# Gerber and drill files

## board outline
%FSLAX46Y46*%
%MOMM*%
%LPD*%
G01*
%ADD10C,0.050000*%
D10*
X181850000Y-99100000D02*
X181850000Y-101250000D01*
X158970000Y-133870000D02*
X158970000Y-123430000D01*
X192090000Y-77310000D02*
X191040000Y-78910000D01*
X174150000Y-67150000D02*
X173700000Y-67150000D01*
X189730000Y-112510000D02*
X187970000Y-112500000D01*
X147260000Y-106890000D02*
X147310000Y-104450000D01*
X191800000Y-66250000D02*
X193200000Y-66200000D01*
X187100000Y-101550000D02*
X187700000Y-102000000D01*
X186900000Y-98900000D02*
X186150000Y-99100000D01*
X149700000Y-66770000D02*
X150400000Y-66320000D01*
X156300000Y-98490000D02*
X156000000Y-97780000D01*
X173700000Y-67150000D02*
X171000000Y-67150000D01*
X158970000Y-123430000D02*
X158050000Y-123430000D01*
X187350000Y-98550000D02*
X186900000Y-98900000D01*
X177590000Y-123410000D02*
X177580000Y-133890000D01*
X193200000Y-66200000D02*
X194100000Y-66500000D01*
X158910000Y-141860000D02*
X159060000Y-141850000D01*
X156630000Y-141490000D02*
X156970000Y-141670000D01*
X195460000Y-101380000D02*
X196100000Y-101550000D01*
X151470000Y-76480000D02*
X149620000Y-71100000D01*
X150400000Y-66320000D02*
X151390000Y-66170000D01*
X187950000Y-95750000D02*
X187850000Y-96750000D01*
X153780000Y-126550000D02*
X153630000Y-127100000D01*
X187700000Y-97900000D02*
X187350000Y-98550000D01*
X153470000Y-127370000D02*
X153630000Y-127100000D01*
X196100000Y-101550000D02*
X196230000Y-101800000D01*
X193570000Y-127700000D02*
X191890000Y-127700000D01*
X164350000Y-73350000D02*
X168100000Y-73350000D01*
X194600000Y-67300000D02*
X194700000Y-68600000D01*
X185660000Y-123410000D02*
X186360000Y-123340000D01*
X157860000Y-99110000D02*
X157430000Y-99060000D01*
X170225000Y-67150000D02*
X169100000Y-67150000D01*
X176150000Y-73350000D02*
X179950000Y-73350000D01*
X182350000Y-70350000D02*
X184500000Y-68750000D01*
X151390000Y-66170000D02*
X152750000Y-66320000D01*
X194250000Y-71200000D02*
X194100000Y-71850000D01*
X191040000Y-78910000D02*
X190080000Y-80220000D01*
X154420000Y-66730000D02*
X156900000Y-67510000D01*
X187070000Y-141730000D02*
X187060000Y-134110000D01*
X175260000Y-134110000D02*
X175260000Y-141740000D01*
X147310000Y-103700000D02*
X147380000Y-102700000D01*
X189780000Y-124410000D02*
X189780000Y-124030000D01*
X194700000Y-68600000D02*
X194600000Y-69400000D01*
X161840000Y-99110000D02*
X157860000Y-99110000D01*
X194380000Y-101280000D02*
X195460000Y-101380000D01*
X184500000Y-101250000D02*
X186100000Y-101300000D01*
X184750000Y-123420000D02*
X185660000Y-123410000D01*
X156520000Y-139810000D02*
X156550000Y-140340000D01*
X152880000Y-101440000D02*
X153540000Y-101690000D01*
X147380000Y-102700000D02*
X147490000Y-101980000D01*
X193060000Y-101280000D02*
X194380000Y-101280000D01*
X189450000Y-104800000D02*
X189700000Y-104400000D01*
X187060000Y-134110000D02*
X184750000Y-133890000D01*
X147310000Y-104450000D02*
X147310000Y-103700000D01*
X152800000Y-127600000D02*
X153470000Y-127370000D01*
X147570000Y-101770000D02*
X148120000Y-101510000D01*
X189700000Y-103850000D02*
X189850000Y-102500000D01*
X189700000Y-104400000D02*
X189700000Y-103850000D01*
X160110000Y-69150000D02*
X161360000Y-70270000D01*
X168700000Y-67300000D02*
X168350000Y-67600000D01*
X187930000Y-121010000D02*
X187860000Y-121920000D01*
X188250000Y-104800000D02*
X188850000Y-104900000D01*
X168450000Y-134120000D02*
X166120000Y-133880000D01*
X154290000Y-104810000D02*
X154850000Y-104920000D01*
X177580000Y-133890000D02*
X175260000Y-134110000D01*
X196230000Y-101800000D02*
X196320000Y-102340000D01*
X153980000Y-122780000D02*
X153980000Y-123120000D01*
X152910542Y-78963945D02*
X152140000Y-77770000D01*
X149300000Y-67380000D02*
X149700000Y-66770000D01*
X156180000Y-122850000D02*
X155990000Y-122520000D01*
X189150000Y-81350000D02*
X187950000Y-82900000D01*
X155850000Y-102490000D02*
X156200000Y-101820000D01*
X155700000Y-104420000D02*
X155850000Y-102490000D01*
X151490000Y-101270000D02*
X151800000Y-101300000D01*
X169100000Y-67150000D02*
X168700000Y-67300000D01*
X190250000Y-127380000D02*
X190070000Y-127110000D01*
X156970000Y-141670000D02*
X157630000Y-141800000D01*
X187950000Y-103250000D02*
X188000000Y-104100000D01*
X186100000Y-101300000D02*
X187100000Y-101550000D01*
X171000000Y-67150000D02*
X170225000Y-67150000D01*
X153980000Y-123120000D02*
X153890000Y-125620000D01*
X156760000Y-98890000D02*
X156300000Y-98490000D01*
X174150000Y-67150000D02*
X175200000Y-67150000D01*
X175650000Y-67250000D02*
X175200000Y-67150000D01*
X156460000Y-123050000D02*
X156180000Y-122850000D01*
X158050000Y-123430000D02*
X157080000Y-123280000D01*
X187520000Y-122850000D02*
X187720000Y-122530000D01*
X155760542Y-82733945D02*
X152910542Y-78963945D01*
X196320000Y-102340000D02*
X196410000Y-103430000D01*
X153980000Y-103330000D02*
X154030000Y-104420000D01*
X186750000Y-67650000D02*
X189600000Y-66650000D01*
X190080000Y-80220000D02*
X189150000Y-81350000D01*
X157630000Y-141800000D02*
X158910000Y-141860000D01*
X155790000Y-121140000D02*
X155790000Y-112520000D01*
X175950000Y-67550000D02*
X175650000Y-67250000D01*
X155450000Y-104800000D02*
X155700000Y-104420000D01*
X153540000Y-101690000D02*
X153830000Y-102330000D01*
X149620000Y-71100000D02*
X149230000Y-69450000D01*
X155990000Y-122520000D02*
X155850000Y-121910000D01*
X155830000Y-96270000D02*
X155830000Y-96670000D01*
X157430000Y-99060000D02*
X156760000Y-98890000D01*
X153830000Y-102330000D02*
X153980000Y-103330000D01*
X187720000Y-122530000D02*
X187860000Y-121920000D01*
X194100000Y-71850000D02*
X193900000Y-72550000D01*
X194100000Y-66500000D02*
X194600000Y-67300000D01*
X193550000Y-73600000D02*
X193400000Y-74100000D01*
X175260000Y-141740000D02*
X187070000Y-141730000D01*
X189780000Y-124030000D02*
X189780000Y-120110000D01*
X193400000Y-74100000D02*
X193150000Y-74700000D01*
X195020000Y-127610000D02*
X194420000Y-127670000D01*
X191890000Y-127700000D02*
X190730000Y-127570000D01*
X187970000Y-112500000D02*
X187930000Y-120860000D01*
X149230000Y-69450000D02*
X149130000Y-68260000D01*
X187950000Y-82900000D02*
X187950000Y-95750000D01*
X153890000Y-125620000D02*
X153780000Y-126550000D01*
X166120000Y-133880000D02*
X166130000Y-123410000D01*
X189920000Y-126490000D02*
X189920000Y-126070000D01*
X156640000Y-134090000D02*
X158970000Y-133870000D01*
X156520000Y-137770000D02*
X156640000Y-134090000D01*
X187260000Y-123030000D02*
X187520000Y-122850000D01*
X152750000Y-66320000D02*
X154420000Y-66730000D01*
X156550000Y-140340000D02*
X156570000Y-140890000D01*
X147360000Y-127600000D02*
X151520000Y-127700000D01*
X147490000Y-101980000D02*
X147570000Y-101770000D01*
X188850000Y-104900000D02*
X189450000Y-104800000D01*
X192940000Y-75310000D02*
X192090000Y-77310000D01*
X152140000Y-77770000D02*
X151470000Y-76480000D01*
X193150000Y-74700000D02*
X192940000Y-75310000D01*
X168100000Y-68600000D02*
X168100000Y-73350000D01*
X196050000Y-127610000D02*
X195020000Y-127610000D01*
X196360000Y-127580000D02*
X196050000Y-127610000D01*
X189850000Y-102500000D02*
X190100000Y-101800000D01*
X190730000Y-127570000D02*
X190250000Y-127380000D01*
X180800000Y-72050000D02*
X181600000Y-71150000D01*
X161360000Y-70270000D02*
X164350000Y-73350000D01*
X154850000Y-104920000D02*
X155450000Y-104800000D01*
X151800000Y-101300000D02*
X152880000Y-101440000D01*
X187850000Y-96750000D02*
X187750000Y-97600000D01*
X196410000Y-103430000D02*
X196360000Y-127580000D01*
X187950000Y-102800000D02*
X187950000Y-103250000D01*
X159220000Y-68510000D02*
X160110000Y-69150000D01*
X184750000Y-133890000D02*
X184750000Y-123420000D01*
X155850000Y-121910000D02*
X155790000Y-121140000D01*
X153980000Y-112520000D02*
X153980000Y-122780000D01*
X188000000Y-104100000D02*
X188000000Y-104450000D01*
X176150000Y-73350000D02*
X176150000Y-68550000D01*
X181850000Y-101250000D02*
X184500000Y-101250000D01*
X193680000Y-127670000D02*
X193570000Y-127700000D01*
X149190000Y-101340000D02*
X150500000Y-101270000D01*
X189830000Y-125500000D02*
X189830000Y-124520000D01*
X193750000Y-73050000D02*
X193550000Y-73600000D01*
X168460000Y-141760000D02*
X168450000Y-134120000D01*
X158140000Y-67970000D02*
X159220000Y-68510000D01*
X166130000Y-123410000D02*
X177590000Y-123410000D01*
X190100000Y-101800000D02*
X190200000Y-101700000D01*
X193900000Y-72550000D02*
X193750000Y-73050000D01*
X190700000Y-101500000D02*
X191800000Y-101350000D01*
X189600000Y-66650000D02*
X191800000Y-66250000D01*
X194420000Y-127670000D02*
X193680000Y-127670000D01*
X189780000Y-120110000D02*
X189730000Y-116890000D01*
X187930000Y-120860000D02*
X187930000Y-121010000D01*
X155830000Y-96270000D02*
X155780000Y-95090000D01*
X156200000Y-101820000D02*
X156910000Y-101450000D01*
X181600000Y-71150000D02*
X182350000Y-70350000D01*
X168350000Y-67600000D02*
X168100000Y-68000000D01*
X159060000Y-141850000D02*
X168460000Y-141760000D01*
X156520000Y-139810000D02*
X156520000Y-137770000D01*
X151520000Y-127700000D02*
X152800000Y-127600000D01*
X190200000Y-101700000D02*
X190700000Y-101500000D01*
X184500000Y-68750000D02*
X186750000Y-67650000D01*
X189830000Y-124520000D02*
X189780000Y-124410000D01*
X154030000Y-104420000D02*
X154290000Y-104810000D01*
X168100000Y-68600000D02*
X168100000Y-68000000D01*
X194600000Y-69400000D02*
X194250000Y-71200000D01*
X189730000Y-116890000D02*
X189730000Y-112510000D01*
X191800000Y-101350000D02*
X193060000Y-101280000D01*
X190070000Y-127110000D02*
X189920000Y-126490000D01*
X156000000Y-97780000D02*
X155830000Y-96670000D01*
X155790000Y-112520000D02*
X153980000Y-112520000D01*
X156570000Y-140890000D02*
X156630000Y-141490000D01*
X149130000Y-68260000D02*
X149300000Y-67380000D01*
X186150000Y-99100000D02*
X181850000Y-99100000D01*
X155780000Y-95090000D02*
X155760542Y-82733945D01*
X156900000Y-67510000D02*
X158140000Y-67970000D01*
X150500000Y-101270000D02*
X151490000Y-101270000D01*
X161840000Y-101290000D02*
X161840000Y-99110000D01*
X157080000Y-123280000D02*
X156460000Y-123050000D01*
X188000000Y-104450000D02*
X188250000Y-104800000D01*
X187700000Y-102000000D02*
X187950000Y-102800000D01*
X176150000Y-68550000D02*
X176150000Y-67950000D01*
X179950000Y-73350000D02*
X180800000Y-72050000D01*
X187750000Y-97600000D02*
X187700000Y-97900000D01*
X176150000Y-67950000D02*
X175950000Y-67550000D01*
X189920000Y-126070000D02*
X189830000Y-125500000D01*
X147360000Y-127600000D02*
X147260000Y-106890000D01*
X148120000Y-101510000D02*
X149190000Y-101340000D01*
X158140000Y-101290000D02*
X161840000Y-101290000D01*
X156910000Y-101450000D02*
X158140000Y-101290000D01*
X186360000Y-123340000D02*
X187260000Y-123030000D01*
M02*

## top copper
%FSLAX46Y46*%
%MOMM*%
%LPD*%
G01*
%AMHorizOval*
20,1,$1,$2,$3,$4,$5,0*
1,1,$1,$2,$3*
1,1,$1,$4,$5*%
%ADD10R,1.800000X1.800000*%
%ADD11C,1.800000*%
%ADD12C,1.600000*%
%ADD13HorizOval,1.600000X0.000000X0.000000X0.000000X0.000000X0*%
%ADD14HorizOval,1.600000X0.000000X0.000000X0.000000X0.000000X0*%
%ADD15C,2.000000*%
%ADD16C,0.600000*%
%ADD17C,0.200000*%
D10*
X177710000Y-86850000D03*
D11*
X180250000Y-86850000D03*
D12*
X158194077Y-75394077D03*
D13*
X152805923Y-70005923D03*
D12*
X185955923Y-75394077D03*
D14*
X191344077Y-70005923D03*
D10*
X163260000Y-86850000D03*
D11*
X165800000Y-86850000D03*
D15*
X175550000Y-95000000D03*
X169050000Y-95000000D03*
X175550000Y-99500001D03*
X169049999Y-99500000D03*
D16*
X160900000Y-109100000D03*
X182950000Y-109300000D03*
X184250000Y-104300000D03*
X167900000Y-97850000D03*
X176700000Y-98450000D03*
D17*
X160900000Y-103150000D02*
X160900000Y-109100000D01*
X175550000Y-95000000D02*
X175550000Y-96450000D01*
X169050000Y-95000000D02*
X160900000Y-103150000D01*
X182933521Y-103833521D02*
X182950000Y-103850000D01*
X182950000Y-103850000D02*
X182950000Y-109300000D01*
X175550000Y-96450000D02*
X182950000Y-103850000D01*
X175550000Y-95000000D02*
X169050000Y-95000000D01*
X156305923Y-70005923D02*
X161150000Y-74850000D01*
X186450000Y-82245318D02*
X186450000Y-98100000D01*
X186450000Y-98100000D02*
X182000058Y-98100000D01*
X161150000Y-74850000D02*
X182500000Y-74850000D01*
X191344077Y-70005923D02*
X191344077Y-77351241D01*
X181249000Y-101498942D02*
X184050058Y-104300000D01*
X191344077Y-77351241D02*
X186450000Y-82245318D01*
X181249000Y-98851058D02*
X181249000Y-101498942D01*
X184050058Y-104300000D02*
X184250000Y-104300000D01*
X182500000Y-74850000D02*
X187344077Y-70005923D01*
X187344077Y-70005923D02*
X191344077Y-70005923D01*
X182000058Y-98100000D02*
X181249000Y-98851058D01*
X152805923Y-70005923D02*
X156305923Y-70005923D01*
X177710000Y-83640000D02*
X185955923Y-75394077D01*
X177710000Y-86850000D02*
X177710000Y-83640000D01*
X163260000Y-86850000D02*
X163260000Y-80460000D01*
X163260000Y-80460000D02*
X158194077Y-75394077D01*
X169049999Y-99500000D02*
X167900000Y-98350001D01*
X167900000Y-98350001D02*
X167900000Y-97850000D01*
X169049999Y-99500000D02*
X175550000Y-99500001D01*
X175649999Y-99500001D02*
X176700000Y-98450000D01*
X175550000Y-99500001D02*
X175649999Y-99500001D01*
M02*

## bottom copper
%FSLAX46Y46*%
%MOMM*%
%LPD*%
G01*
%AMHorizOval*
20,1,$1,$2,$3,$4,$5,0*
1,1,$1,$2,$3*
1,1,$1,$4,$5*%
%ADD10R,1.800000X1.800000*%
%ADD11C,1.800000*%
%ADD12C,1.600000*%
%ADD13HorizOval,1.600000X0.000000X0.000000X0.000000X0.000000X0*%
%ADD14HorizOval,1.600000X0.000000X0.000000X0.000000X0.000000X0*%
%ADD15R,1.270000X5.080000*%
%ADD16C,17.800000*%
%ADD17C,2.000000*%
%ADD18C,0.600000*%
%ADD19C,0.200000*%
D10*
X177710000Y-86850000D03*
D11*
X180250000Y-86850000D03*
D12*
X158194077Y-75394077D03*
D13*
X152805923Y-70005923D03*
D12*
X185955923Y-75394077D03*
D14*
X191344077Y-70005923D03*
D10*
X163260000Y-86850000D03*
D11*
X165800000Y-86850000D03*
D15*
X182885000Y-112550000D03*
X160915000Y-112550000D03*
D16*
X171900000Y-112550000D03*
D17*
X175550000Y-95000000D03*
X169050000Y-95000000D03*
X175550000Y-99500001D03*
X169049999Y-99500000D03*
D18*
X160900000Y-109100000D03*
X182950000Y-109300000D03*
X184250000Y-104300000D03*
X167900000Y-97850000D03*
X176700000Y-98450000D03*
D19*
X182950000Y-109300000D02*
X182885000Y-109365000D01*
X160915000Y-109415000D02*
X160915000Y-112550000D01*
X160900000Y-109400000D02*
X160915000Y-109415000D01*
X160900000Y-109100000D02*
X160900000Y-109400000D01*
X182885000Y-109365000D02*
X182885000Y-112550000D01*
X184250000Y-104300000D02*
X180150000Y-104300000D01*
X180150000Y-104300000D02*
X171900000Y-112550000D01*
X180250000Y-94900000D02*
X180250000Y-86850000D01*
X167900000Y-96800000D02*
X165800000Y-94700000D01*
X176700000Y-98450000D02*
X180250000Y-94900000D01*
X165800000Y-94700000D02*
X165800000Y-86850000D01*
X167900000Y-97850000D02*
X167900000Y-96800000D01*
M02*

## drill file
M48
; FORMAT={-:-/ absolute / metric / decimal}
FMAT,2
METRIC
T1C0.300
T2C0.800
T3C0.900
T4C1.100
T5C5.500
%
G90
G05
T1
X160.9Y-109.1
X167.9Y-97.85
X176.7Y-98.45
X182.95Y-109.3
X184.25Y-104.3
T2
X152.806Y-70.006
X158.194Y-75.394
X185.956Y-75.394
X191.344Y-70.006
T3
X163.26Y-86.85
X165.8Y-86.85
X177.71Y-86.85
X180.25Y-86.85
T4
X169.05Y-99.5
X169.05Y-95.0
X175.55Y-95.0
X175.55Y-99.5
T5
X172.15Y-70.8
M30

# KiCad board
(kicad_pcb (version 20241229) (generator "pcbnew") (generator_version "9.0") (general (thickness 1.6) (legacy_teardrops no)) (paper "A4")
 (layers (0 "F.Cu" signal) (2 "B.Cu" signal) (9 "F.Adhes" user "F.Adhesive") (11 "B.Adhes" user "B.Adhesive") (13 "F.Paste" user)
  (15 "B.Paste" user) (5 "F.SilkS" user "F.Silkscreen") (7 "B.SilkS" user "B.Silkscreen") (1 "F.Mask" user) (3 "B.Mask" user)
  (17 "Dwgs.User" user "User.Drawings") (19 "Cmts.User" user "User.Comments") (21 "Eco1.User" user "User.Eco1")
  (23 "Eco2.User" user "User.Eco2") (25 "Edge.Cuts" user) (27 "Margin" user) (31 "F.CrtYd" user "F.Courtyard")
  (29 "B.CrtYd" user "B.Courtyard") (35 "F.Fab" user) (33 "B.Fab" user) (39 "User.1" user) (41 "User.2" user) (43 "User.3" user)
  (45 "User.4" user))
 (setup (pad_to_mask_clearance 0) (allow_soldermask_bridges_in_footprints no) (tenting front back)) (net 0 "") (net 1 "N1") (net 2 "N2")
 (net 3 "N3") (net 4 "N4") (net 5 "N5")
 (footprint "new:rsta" (layer "F.Cu") (at 170.3 106.931432)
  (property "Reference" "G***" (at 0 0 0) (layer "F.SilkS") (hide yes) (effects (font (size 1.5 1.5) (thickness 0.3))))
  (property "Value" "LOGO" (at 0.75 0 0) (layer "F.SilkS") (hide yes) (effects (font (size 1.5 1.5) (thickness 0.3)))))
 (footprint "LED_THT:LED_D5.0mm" (layer "F.Cu") (at 177.71 86.85)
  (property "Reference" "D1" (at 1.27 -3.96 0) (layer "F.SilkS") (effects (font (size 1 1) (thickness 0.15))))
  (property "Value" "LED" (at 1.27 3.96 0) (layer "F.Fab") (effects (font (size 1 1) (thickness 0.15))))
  (pad "1" thru_hole rect (at 0 0) (size 1.8 1.8) (drill 0.9) (layers "*.Cu" "*.Mask") (remove_unused_layers no) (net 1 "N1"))
  (pad "2" thru_hole circle (at 2.54 0) (size 1.8 1.8) (drill 0.9) (layers "*.Cu" "*.Mask") (remove_unused_layers no) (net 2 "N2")))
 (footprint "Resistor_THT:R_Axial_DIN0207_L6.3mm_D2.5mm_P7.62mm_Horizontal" (layer "F.Cu") (at 158.194077 75.394077 135)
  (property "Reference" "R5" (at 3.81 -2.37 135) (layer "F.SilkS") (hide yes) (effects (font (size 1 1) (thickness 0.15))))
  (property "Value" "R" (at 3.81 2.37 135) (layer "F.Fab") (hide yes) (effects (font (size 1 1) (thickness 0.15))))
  (pad "1" thru_hole circle (at 0 0 135) (size 1.6 1.6) (drill 0.8) (layers "*.Cu" "*.Mask") (remove_unused_layers no) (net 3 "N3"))
  (pad "2" thru_hole oval (at 7.62 0 135) (size 1.6 1.6) (drill 0.8) (layers "*.Cu" "*.Mask") (remove_unused_layers no) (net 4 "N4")))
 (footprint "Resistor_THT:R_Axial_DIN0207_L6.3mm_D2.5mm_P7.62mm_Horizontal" (layer "F.Cu") (at 185.955923 75.394077 45)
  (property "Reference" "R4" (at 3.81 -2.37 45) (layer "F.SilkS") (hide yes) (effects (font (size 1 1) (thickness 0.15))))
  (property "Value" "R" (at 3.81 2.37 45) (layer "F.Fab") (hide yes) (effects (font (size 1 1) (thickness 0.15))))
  (pad "1" thru_hole circle (at 0 0 45) (size 1.6 1.6) (drill 0.8) (layers "*.Cu" "*.Mask") (remove_unused_layers no) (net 1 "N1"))
  (pad "2" thru_hole oval (at 7.62 0 45) (size 1.6 1.6) (drill 0.8) (layers "*.Cu" "*.Mask") (remove_unused_layers no) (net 4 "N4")))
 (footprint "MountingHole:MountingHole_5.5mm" (layer "F.Cu") (at 172.15 70.8)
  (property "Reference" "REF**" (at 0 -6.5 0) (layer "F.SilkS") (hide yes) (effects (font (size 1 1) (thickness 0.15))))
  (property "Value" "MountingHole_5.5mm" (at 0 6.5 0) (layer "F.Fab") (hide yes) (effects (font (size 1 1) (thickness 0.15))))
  (pad "" np_thru_hole circle (at 0 0) (size 5.5 5.5) (drill 5.5) (layers "*.Cu" "*.Mask")))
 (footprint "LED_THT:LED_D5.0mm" (layer "F.Cu") (at 163.26 86.85)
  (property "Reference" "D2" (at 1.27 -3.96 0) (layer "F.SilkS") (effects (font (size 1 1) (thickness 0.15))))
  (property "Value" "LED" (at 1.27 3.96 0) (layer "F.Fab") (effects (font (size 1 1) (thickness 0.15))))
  (pad "1" thru_hole rect (at 0 0) (size 1.8 1.8) (drill 0.9) (layers "*.Cu" "*.Mask") (remove_unused_layers no) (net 3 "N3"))
  (pad "2" thru_hole circle (at 2.54 0) (size 1.8 1.8) (drill 0.9) (layers "*.Cu" "*.Mask") (remove_unused_layers no) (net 2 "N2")))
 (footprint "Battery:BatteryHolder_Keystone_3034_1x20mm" (layer "B.Cu") (at 171.9 112.55 180)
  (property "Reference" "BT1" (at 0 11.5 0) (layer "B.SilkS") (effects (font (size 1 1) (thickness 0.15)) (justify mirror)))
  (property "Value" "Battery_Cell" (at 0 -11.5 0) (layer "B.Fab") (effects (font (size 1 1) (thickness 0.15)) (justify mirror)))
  (pad "1" smd rect (at -10.985 0 180) (size 1.27 5.08) (layers "B.Cu" "B.Mask" "B.Paste") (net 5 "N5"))
  (pad "1" smd rect (at 10.985 0 180) (size 1.27 5.08) (layers "B.Cu" "B.Mask" "B.Paste") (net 5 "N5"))
  (pad "2" smd circle (at 0 0 180) (size 17.8 17.8) (layers "B.Cu" "B.Mask") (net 4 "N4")))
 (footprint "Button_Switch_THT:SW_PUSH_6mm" (layer "B.Cu") (at 175.55 95 180)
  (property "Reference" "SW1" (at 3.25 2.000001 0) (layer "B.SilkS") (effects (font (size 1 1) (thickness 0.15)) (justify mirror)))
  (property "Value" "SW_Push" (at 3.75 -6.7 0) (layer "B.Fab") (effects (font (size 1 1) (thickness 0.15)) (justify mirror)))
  (pad "1" thru_hole circle (at 0 0 90) (size 2 2) (drill 1.1) (layers "*.Cu" "*.Mask") (remove_unused_layers no) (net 5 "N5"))
  (pad "1" thru_hole circle (at 6.5 0 90) (size 2 2) (drill 1.1) (layers "*.Cu" "*.Mask") (remove_unused_layers no) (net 5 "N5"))
  (pad "2" thru_hole circle (at 0 -4.500001 90) (size 2 2) (drill 1.1) (layers "*.Cu" "*.Mask") (remove_unused_layers no) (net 2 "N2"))
  (pad "2" thru_hole circle (at 6.500001 -4.5 90) (size 2 2) (drill 1.1) (layers "*.Cu" "*.Mask") (remove_unused_layers no) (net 2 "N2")))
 (gr_line (start 181.85 99.1) (end 181.85 101.25) (stroke (width 0.05) (type default)) (layer "Edge.Cuts"))
 (gr_line (start 158.97 133.87) (end 158.97 123.43) (stroke (width 0.05) (type default)) (layer "Edge.Cuts"))
 (gr_line (start 192.09 77.31) (end 191.04 78.91) (stroke (width 0.05) (type default)) (layer "Edge.Cuts"))
 (gr_line (start 174.15 67.15) (end 173.7 67.15) (stroke (width 0.05) (type default)) (layer "Edge.Cuts"))
 (gr_line (start 189.73 112.51) (end 187.97 112.5) (stroke (width 0.05) (type default)) (layer "Edge.Cuts"))
 (gr_line (start 147.26 106.89) (end 147.31 104.45) (stroke (width 0.05) (type default)) (layer "Edge.Cuts"))
 (gr_line (start 191.8 66.25) (end 193.2 66.2) (stroke (width 0.05) (type default)) (layer "Edge.Cuts"))
 (gr_line (start 187.1 101.55) (end 187.7 102) (stroke (width 0.05) (type default)) (layer "Edge.Cuts"))
 (gr_line (start 186.9 98.9) (end 186.15 99.1) (stroke (width 0.05) (type default)) (layer "Edge.Cuts"))
 (gr_line (start 149.7 66.77) (end 150.4 66.32) (stroke (width 0.05) (type default)) (layer "Edge.Cuts"))
 (gr_line (start 156.3 98.49) (end 156 97.78) (stroke (width 0.05) (type default)) (layer "Edge.Cuts"))
 (gr_line (start 173.7 67.15) (end 171 67.15) (stroke (width 0.05) (type default)) (layer "Edge.Cuts"))
 (gr_line (start 158.97 123.43) (end 158.05 123.43) (stroke (width 0.05) (type default)) (layer "Edge.Cuts"))
 (gr_line (start 187.35 98.55) (end 186.9 98.9) (stroke (width 0.05) (type default)) (layer "Edge.Cuts"))
 (gr_line (start 177.59 123.41) (end 177.58 133.89) (stroke (width 0.05) (type default)) (layer "Edge.Cuts"))
 (gr_line (start 193.2 66.2) (end 194.1 66.5) (stroke (width 0.05) (type default)) (layer "Edge.Cuts"))
 (gr_line (start 158.91 141.86) (end 159.06 141.85) (stroke (width 0.05) (type default)) (layer "Edge.Cuts"))
 (gr_line (start 156.63 141.49) (end 156.97 141.67) (stroke (width 0.05) (type default)) (layer "Edge.Cuts"))
 (gr_line (start 195.46 101.38) (end 196.1 101.55) (stroke (width 0.05) (type default)) (layer "Edge.Cuts"))
 (gr_line (start 151.47 76.48) (end 149.62 71.1) (stroke (width 0.05) (type default)) (layer "Edge.Cuts"))
 (gr_line (start 150.4 66.32) (end 151.39 66.17) (stroke (width 0.05) (type default)) (layer "Edge.Cuts"))
 (gr_line (start 187.95 95.75) (end 187.85 96.75) (stroke (width 0.05) (type default)) (layer "Edge.Cuts"))
 (gr_line (start 153.78 126.55) (end 153.63 127.1) (stroke (width 0.05) (type default)) (layer "Edge.Cuts"))
 (gr_line (start 187.7 97.9) (end 187.35 98.55) (stroke (width 0.05) (type default)) (layer "Edge.Cuts"))
 (gr_line (start 153.47 127.37) (end 153.63 127.1) (stroke (width 0.05) (type default)) (layer "Edge.Cuts"))
 (gr_line (start 196.1 101.55) (end 196.23 101.8) (stroke (width 0.05) (type default)) (layer "Edge.Cuts"))
 (gr_line (start 193.57 127.7) (end 191.89 127.7) (stroke (width 0.05) (type default)) (layer "Edge.Cuts"))
 (gr_line (start 164.35 73.35) (end 168.1 73.35) (stroke (width 0.05) (type default)) (layer "Edge.Cuts"))
 (gr_line (start 194.6 67.3) (end 194.7 68.6) (stroke (width 0.05) (type default)) (layer "Edge.Cuts"))
 (gr_line (start 185.66 123.41) (end 186.36 123.34) (stroke (width 0.05) (type default)) (layer "Edge.Cuts"))
 (gr_line (start 157.86 99.11) (end 157.43 99.06) (stroke (width 0.05) (type default)) (layer "Edge.Cuts"))
 (gr_line (start 170.225 67.15) (end 169.1 67.15) (stroke (width 0.05) (type default)) (layer "Edge.Cuts"))
 (gr_line (start 176.15 73.35) (end 179.95 73.35) (stroke (width 0.05) (type default)) (layer "Edge.Cuts"))
 (gr_line (start 182.35 70.35) (end 184.5 68.75) (stroke (width 0.05) (type default)) (layer "Edge.Cuts"))
 (gr_line (start 151.39 66.17) (end 152.75 66.32) (stroke (width 0.05) (type default)) (layer "Edge.Cuts"))
 (gr_line (start 194.25 71.2) (end 194.1 71.85) (stroke (width 0.05) (type default)) (layer "Edge.Cuts"))
 (gr_line (start 191.04 78.91) (end 190.08 80.22) (stroke (width 0.05) (type default)) (layer "Edge.Cuts"))
 (gr_line (start 154.42 66.73) (end 156.9 67.51) (stroke (width 0.05) (type default)) (layer "Edge.Cuts"))
 (gr_line (start 187.07 141.73) (end 187.06 134.11) (stroke (width 0.05) (type default)) (layer "Edge.Cuts"))
 (gr_line (start 175.26 134.11) (end 175.26 141.74) (stroke (width 0.05) (type default)) (layer "Edge.Cuts"))
 (gr_line (start 147.31 103.7) (end 147.38 102.7) (stroke (width 0.05) (type default)) (layer "Edge.Cuts"))
 (gr_line (start 189.78 124.41) (end 189.78 124.03) (stroke (width 0.05) (type default)) (layer "Edge.Cuts"))
 (gr_line (start 194.7 68.6) (end 194.6 69.4) (stroke (width 0.05) (type default)) (layer "Edge.Cuts"))
 (gr_line (start 161.84 99.11) (end 157.86 99.11) (stroke (width 0.05) (type default)) (layer "Edge.Cuts"))
 (gr_line (start 194.38 101.28) (end 195.46 101.38) (stroke (width 0.05) (type default)) (layer "Edge.Cuts"))
 (gr_line (start 184.5 101.25) (end 186.1 101.3) (stroke (width 0.05) (type default)) (layer "Edge.Cuts"))
 (gr_line (start 184.75 123.42) (end 185.66 123.41) (stroke (width 0.05) (type default)) (layer "Edge.Cuts"))
 (gr_line (start 156.52 139.81) (end 156.55 140.34) (stroke (width 0.05) (type default)) (layer "Edge.Cuts"))
 (gr_line (start 152.88 101.44) (end 153.54 101.69) (stroke (width 0.05) (type default)) (layer "Edge.Cuts"))
 (gr_line (start 147.38 102.7) (end 147.49 101.98) (stroke (width 0.05) (type default)) (layer "Edge.Cuts"))
 (gr_line (start 193.06 101.28) (end 194.38 101.28) (stroke (width 0.05) (type default)) (layer "Edge.Cuts"))
 (gr_line (start 189.45 104.8) (end 189.7 104.4) (stroke (width 0.05) (type default)) (layer "Edge.Cuts"))
 (gr_line (start 187.06 134.11) (end 184.75 133.89) (stroke (width 0.05) (type default)) (layer "Edge.Cuts"))
 (gr_line (start 147.31 104.45) (end 147.31 103.7) (stroke (width 0.05) (type default)) (layer "Edge.Cuts"))
 (gr_line (start 152.8 127.6) (end 153.47 127.37) (stroke (width 0.05) (type default)) (layer "Edge.Cuts"))
 (gr_line (start 147.57 101.77) (end 148.12 101.51) (stroke (width 0.05) (type default)) (layer "Edge.Cuts"))
 (gr_line (start 189.7 103.85) (end 189.85 102.5) (stroke (width 0.05) (type default)) (layer "Edge.Cuts"))
 (gr_line (start 189.7 104.4) (end 189.7 103.85) (stroke (width 0.05) (type default)) (layer "Edge.Cuts"))
 (gr_line (start 160.11 69.15) (end 161.36 70.27) (stroke (width 0.05) (type default)) (layer "Edge.Cuts"))
 (gr_line (start 168.7 67.3) (end 168.35 67.6) (stroke (width 0.05) (type default)) (layer "Edge.Cuts"))
 (gr_line (start 187.93 121.01) (end 187.86 121.92) (stroke (width 0.05) (type default)) (layer "Edge.Cuts"))
 (gr_line (start 188.25 104.8) (end 188.85 104.9) (stroke (width 0.05) (type default)) (layer "Edge.Cuts"))
 (gr_line (start 168.45 134.12) (end 166.12 133.88) (stroke (width 0.05) (type default)) (layer "Edge.Cuts"))
 (gr_line (start 154.29 104.81) (end 154.85 104.92) (stroke (width 0.05) (type default)) (layer "Edge.Cuts"))
 (gr_line (start 177.58 133.89) (end 175.26 134.11) (stroke (width 0.05) (type default)) (layer "Edge.Cuts"))
 (gr_line (start 196.23 101.8) (end 196.32 102.34) (stroke (width 0.05) (type default)) (layer "Edge.Cuts"))
 (gr_line (start 153.98 122.78) (end 153.98 123.12) (stroke (width 0.05) (type default)) (layer "Edge.Cuts"))
 (gr_line (start 152.910542 78.963945) (end 152.14 77.77) (stroke (width 0.05) (type default)) (layer "Edge.Cuts"))
 (gr_line (start 149.3 67.38) (end 149.7 66.77) (stroke (width 0.05) (type default)) (layer "Edge.Cuts"))
 (gr_line (start 156.18 122.85) (end 155.99 122.52) (stroke (width 0.05) (type default)) (layer "Edge.Cuts"))
 (gr_line (start 189.15 81.35) (end 187.95 82.9) (stroke (width 0.05) (type default)) (layer "Edge.Cuts"))
 (gr_line (start 155.85 102.49) (end 156.2 101.82) (stroke (width 0.05) (type default)) (layer "Edge.Cuts"))
 (gr_line (start 155.7 104.42) (end 155.85 102.49) (stroke (width 0.05) (type default)) (layer "Edge.Cuts"))
 (gr_line (start 151.49 101.27) (end 151.8 101.3) (stroke (width 0.05) (type default)) (layer "Edge.Cuts"))
 (gr_line (start 169.1 67.15) (end 168.7 67.3) (stroke (width 0.05) (type default)) (layer "Edge.Cuts"))
 (gr_line (start 190.25 127.38) (end 190.07 127.11) (stroke (width 0.05) (type default)) (layer "Edge.Cuts"))
 (gr_line (start 156.97 141.67) (end 157.63 141.8) (stroke (width 0.05) (type default)) (layer "Edge.Cuts"))
 (gr_line (start 187.95 103.25) (end 188 104.1) (stroke (width 0.05) (type default)) (layer "Edge.Cuts"))
 (gr_line (start 186.1 101.3) (end 187.1 101.55) (stroke (width 0.05) (type default)) (layer "Edge.Cuts"))
 (gr_line (start 171 67.15) (end 170.225 67.15) (stroke (width 0.05) (type default)) (layer "Edge.Cuts"))
 (gr_line (start 153.98 123.12) (end 153.89 125.62) (stroke (width 0.05) (type default)) (layer "Edge.Cuts"))
 (gr_line (start 156.76 98.89) (end 156.3 98.49) (stroke (width 0.05) (type default)) (layer "Edge.Cuts"))
 (gr_line (start 174.15 67.15) (end 175.2 67.15) (stroke (width 0.05) (type default)) (layer "Edge.Cuts"))
 (gr_line (start 175.65 67.25) (end 175.2 67.15) (stroke (width 0.05) (type default)) (layer "Edge.Cuts"))
 (gr_line (start 156.46 123.05) (end 156.18 122.85) (stroke (width 0.05) (type default)) (layer "Edge.Cuts"))
 (gr_line (start 158.05 123.43) (end 157.08 123.28) (stroke (width 0.05) (type default)) (layer "Edge.Cuts"))
 (gr_line (start 187.52 122.85) (end 187.72 122.53) (stroke (width 0.05) (type default)) (layer "Edge.Cuts"))
 (gr_line (start 155.760542 82.733945) (end 152.910542 78.963945) (stroke (width 0.05) (type default)) (layer "Edge.Cuts"))
 (gr_line (start 196.32 102.34) (end 196.41 103.43) (stroke (width 0.05) (type default)) (layer "Edge.Cuts"))
 (gr_line (start 153.98 103.33) (end 154.03 104.42) (stroke (width 0.05) (type default)) (layer "Edge.Cuts"))
 (gr_line (start 186.75 67.65) (end 189.6 66.65) (stroke (width 0.05) (type default)) (layer "Edge.Cuts"))
 (gr_line (start 190.08 80.22) (end 189.15 81.35) (stroke (width 0.05) (type default)) (layer "Edge.Cuts"))
 (gr_line (start 157.63 141.8) (end 158.91 141.86) (stroke (width 0.05) (type default)) (layer "Edge.Cuts"))
 (gr_line (start 155.79 121.14) (end 155.79 112.52) (stroke (width 0.05) (type default)) (layer "Edge.Cuts"))
 (gr_line (start 175.95 67.55) (end 175.65 67.25) (stroke (width 0.05) (type default)) (layer "Edge.Cuts"))
 (gr_line (start 155.45 104.8) (end 155.7 104.42) (stroke (width 0.05) (type default)) (layer "Edge.Cuts"))
 (gr_line (start 153.54 101.69) (end 153.83 102.33) (stroke (width 0.05) (type default)) (layer "Edge.Cuts"))
 (gr_line (start 149.62 71.1) (end 149.23 69.45) (stroke (width 0.05) (type default)) (layer "Edge.Cuts"))
 (gr_line (start 155.99 122.52) (end 155.85 121.91) (stroke (width 0.05) (type default)) (layer "Edge.Cuts"))
 (gr_line (start 155.83 96.27) (end 155.83 96.67) (stroke (width 0.05) (type default)) (layer "Edge.Cuts"))
 (gr_line (start 157.43 99.06) (end 156.76 98.89) (stroke (width 0.05) (type default)) (layer "Edge.Cuts"))
 (gr_line (start 153.83 102.33) (end 153.98 103.33) (stroke (width 0.05) (type default)) (layer "Edge.Cuts"))
 (gr_line (start 187.72 122.53) (end 187.86 121.92) (stroke (width 0.05) (type default)) (layer "Edge.Cuts"))
 (gr_line (start 194.1 71.85) (end 193.9 72.55) (stroke (width 0.05) (type default)) (layer "Edge.Cuts"))
 (gr_line (start 194.1 66.5) (end 194.6 67.3) (stroke (width 0.05) (type default)) (layer "Edge.Cuts"))
 (gr_line (start 193.55 73.6) (end 193.4 74.1) (stroke (width 0.05) (type default)) (layer "Edge.Cuts"))
 (gr_line (start 175.26 141.74) (end 187.07 141.73) (stroke (width 0.05) (type default)) (layer "Edge.Cuts"))
 (gr_line (start 189.78 124.03) (end 189.78 120.11) (stroke (width 0.05) (type default)) (layer "Edge.Cuts"))
 (gr_line (start 193.4 74.1) (end 193.15 74.7) (stroke (width 0.05) (type default)) (layer "Edge.Cuts"))
 (gr_line (start 195.02 127.61) (end 194.42 127.67) (stroke (width 0.05) (type default)) (layer "Edge.Cuts"))
 (gr_line (start 191.89 127.7) (end 190.73 127.57) (stroke (width 0.05) (type default)) (layer "Edge.Cuts"))
 (gr_line (start 187.97 112.5) (end 187.93 120.86) (stroke (width 0.05) (type default)) (layer "Edge.Cuts"))
 (gr_line (start 149.23 69.45) (end 149.13 68.26) (stroke (width 0.05) (type default)) (layer "Edge.Cuts"))
 (gr_line (start 187.95 82.9) (end 187.95 95.75) (stroke (width 0.05) (type default)) (layer "Edge.Cuts"))
 (gr_line (start 153.89 125.62) (end 153.78 126.55) (stroke (width 0.05) (type default)) (layer "Edge.Cuts"))
 (gr_line (start 166.12 133.88) (end 166.13 123.41) (stroke (width 0.05) (type default)) (layer "Edge.Cuts"))
 (gr_line (start 189.92 126.49) (end 189.92 126.07) (stroke (width 0.05) (type default)) (layer "Edge.Cuts"))
 (gr_line (start 156.64 134.09) (end 158.97 133.87) (stroke (width 0.05) (type default)) (layer "Edge.Cuts"))
 (gr_line (start 156.52 137.77) (end 156.64 134.09) (stroke (width 0.05) (type default)) (layer "Edge.Cuts"))
 (gr_line (start 187.26 123.03) (end 187.52 122.85) (stroke (width 0.05) (type default)) (layer "Edge.Cuts"))
 (gr_line (start 152.75 66.32) (end 154.42 66.73) (stroke (width 0.05) (type default)) (layer "Edge.Cuts"))
 (gr_line (start 156.55 140.34) (end 156.57 140.89) (stroke (width 0.05) (type default)) (layer "Edge.Cuts"))
 (gr_line (start 147.36 127.6) (end 151.52 127.7) (stroke (width 0.05) (type default)) (layer "Edge.Cuts"))
 (gr_line (start 147.49 101.98) (end 147.57 101.77) (stroke (width 0.05) (type default)) (layer "Edge.Cuts"))
 (gr_line (start 188.85 104.9) (end 189.45 104.8) (stroke (width 0.05) (type default)) (layer "Edge.Cuts"))
 (gr_line (start 192.94 75.31) (end 192.09 77.31) (stroke (width 0.05) (type default)) (layer "Edge.Cuts"))
 (gr_line (start 152.14 77.77) (end 151.47 76.48) (stroke (width 0.05) (type default)) (layer "Edge.Cuts"))
 (gr_line (start 193.15 74.7) (end 192.94 75.31) (stroke (width 0.05) (type default)) (layer "Edge.Cuts"))
 (gr_line (start 168.1 68.6) (end 168.1 73.35) (stroke (width 0.05) (type default)) (layer "Edge.Cuts"))
 (gr_line (start 196.05 127.61) (end 195.02 127.61) (stroke (width 0.05) (type default)) (layer "Edge.Cuts"))
 (gr_line (start 196.36 127.58) (end 196.05 127.61) (stroke (width 0.05) (type default)) (layer "Edge.Cuts"))
 (gr_line (start 189.85 102.5) (end 190.1 101.8) (stroke (width 0.05) (type default)) (layer "Edge.Cuts"))
 (gr_line (start 190.73 127.57) (end 190.25 127.38) (stroke (width 0.05) (type default)) (layer "Edge.Cuts"))
 (gr_line (start 180.8 72.05) (end 181.6 71.15) (stroke (width 0.05) (type default)) (layer "Edge.Cuts"))
 (gr_line (start 161.36 70.27) (end 164.35 73.35) (stroke (width 0.05) (type default)) (layer "Edge.Cuts"))
 (gr_line (start 154.85 104.92) (end 155.45 104.8) (stroke (width 0.05) (type default)) (layer "Edge.Cuts"))
 (gr_line (start 151.8 101.3) (end 152.88 101.44) (stroke (width 0.05) (type default)) (layer "Edge.Cuts"))
 (gr_line (start 187.85 96.75) (end 187.75 97.6) (stroke (width 0.05) (type default)) (layer "Edge.Cuts"))
 (gr_line (start 196.41 103.43) (end 196.36 127.58) (stroke (width 0.05) (type default)) (layer "Edge.Cuts"))
 (gr_line (start 187.95 102.8) (end 187.95 103.25) (stroke (width 0.05) (type default)) (layer "Edge.Cuts"))
 (gr_line (start 159.22 68.51) (end 160.11 69.15) (stroke (width 0.05) (type default)) (layer "Edge.Cuts"))
 (gr_line (start 184.75 133.89) (end 184.75 123.42) (stroke (width 0.05) (type default)) (layer "Edge.Cuts"))
 (gr_line (start 155.85 121.91) (end 155.79 121.14) (stroke (width 0.05) (type default)) (layer "Edge.Cuts"))
 (gr_line (start 153.98 112.52) (end 153.98 122.78) (stroke (width 0.05) (type default)) (layer "Edge.Cuts"))
 (gr_line (start 188 104.1) (end 188 104.45) (stroke (width 0.05) (type default)) (layer "Edge.Cuts"))
 (gr_line (start 176.15 73.35) (end 176.15 68.55) (stroke (width 0.05) (type default)) (layer "Edge.Cuts"))
 (gr_line (start 181.85 101.25) (end 184.5 101.25) (stroke (width 0.05) (type default)) (layer "Edge.Cuts"))
 (gr_line (start 193.68 127.67) (end 193.57 127.7) (stroke (width 0.05) (type default)) (layer "Edge.Cuts"))
 (gr_line (start 149.19 101.34) (end 150.5 101.27) (stroke (width 0.05) (type default)) (layer "Edge.Cuts"))
 (gr_line (start 189.83 125.5) (end 189.83 124.52) (stroke (width 0.05) (type default)) (layer "Edge.Cuts"))
 (gr_line (start 193.75 73.05) (end 193.55 73.6) (stroke (width 0.05) (type default)) (layer "Edge.Cuts"))
 (gr_line (start 168.46 141.76) (end 168.45 134.12) (stroke (width 0.05) (type default)) (layer "Edge.Cuts"))
 (gr_line (start 158.14 67.97) (end 159.22 68.51) (stroke (width 0.05) (type default)) (layer "Edge.Cuts"))
 (gr_line (start 166.13 123.41) (end 177.59 123.41) (stroke (width 0.05) (type default)) (layer "Edge.Cuts"))
 (gr_line (start 190.1 101.8) (end 190.2 101.7) (stroke (width 0.05) (type default)) (layer "Edge.Cuts"))
 (gr_line (start 193.9 72.55) (end 193.75 73.05) (stroke (width 0.05) (type default)) (layer "Edge.Cuts"))
 (gr_line (start 190.7 101.5) (end 191.8 101.35) (stroke (width 0.05) (type default)) (layer "Edge.Cuts"))
 (gr_line (start 189.6 66.65) (end 191.8 66.25) (stroke (width 0.05) (type default)) (layer "Edge.Cuts"))
 (gr_line (start 194.42 127.67) (end 193.68 127.67) (stroke (width 0.05) (type default)) (layer "Edge.Cuts"))
 (gr_line (start 189.78 120.11) (end 189.73 116.89) (stroke (width 0.05) (type default)) (layer "Edge.Cuts"))
 (gr_line (start 187.93 120.86) (end 187.93 121.01) (stroke (width 0.05) (type default)) (layer "Edge.Cuts"))
 (gr_line (start 155.83 96.27) (end 155.78 95.09) (stroke (width 0.05) (type default)) (layer "Edge.Cuts"))
 (gr_line (start 156.2 101.82) (end 156.91 101.45) (stroke (width 0.05) (type default)) (layer "Edge.Cuts"))
 (gr_line (start 181.6 71.15) (end 182.35 70.35) (stroke (width 0.05) (type default)) (layer "Edge.Cuts"))
 (gr_line (start 168.35 67.6) (end 168.1 68) (stroke (width 0.05) (type default)) (layer "Edge.Cuts"))
 (gr_line (start 159.06 141.85) (end 168.46 141.76) (stroke (width 0.05) (type default)) (layer "Edge.Cuts"))
 (gr_line (start 156.52 139.81) (end 156.52 137.77) (stroke (width 0.05) (type default)) (layer "Edge.Cuts"))
 (gr_line (start 151.52 127.7) (end 152.8 127.6) (stroke (width 0.05) (type default)) (layer "Edge.Cuts"))
 (gr_line (start 190.2 101.7) (end 190.7 101.5) (stroke (width 0.05) (type default)) (layer "Edge.Cuts"))
 (gr_line (start 184.5 68.75) (end 186.75 67.65) (stroke (width 0.05) (type default)) (layer "Edge.Cuts"))
 (gr_line (start 189.83 124.52) (end 189.78 124.41) (stroke (width 0.05) (type default)) (layer "Edge.Cuts"))
 (gr_line (start 154.03 104.42) (end 154.29 104.81) (stroke (width 0.05) (type default)) (layer "Edge.Cuts"))
 (gr_line (start 168.1 68.6) (end 168.1 68) (stroke (width 0.05) (type default)) (layer "Edge.Cuts"))
 (gr_line (start 194.6 69.4) (end 194.25 71.2) (stroke (width 0.05) (type default)) (layer "Edge.Cuts"))
 (gr_line (start 189.73 116.89) (end 189.73 112.51) (stroke (width 0.05) (type default)) (layer "Edge.Cuts"))
 (gr_line (start 191.8 101.35) (end 193.06 101.28) (stroke (width 0.05) (type default)) (layer "Edge.Cuts"))
 (gr_line (start 190.07 127.11) (end 189.92 126.49) (stroke (width 0.05) (type default)) (layer "Edge.Cuts"))
 (gr_line (start 156 97.78) (end 155.83 96.67) (stroke (width 0.05) (type default)) (layer "Edge.Cuts"))
 (gr_line (start 155.79 112.52) (end 153.98 112.52) (stroke (width 0.05) (type default)) (layer "Edge.Cuts"))
 (gr_line (start 156.57 140.89) (end 156.63 141.49) (stroke (width 0.05) (type default)) (layer "Edge.Cuts"))
 (gr_line (start 149.13 68.26) (end 149.3 67.38) (stroke (width 0.05) (type default)) (layer "Edge.Cuts"))
 (gr_line (start 186.15 99.1) (end 181.85 99.1) (stroke (width 0.05) (type default)) (layer "Edge.Cuts"))
 (gr_line (start 155.78 95.09) (end 155.760542 82.733945) (stroke (width 0.05) (type default)) (layer "Edge.Cuts"))
 (gr_line (start 156.9 67.51) (end 158.14 67.97) (stroke (width 0.05) (type default)) (layer "Edge.Cuts"))
 (gr_line (start 150.5 101.27) (end 151.49 101.27) (stroke (width 0.05) (type default)) (layer "Edge.Cuts"))
 (gr_line (start 161.84 101.29) (end 161.84 99.11) (stroke (width 0.05) (type default)) (layer "Edge.Cuts"))
 (gr_line (start 157.08 123.28) (end 156.46 123.05) (stroke (width 0.05) (type default)) (layer "Edge.Cuts"))
 (gr_line (start 188 104.45) (end 188.25 104.8) (stroke (width 0.05) (type default)) (layer "Edge.Cuts"))
 (gr_line (start 187.7 102) (end 187.95 102.8) (stroke (width 0.05) (type default)) (layer "Edge.Cuts"))
 (gr_line (start 176.15 68.55) (end 176.15 67.95) (stroke (width 0.05) (type default)) (layer "Edge.Cuts"))
 (gr_line (start 179.95 73.35) (end 180.8 72.05) (stroke (width 0.05) (type default)) (layer "Edge.Cuts"))
 (gr_line (start 187.75 97.6) (end 187.7 97.9) (stroke (width 0.05) (type default)) (layer "Edge.Cuts"))
 (gr_line (start 176.15 67.95) (end 175.95 67.55) (stroke (width 0.05) (type default)) (layer "Edge.Cuts"))
 (gr_line (start 189.92 126.07) (end 189.83 125.5) (stroke (width 0.05) (type default)) (layer "Edge.Cuts"))
 (gr_line (start 147.36 127.6) (end 147.26 106.89) (stroke (width 0.05) (type default)) (layer "Edge.Cuts"))
 (gr_line (start 148.12 101.51) (end 149.19 101.34) (stroke (width 0.05) (type default)) (layer "Edge.Cuts"))
 (gr_line (start 158.14 101.29) (end 161.84 101.29) (stroke (width 0.05) (type default)) (layer "Edge.Cuts"))
 (gr_line (start 156.91 101.45) (end 158.14 101.29) (stroke (width 0.05) (type default)) (layer "Edge.Cuts"))
 (gr_line (start 186.36 123.34) (end 187.26 123.03) (stroke (width 0.05) (type default)) (layer "Edge.Cuts"))
 (segment (start 160.9 103.15) (end 160.9 109.1) (width 0.2) (layer "F.Cu") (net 5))
 (segment (start 175.55 95) (end 175.55 96.45) (width 0.2) (layer "F.Cu") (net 5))
 (segment (start 169.05 95) (end 160.9 103.15) (width 0.2) (layer "F.Cu") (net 5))
 (segment (start 182.933521 103.833521) (end 182.95 103.85) (width 0.2) (layer "F.Cu") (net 5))
 (segment (start 182.95 103.85) (end 182.95 109.3) (width 0.2) (layer "F.Cu") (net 5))
 (segment (start 175.55 96.45) (end 182.95 103.85) (width 0.2) (layer "F.Cu") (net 5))
 (segment (start 175.55 95) (end 169.05 95) (width 0.2) (layer "F.Cu") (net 5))
 (via (at 160.9 109.1) (size 0.6) (drill 0.3) (layers "F.Cu" "B.Cu") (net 5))
 (via (at 182.95 109.3) (size 0.6) (drill 0.3) (layers "F.Cu" "B.Cu") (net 5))
 (segment (start 182.95 109.3) (end 182.885 109.365) (width 0.2) (layer "B.Cu") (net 5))
 (segment (start 160.915 109.415) (end 160.915 112.55) (width 0.2) (layer "B.Cu") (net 5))
 (segment (start 160.9 109.4) (end 160.915 109.415) (width 0.2) (layer "B.Cu") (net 5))
 (segment (start 160.9 109.1) (end 160.9 109.4) (width 0.2) (layer "B.Cu") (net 5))
 (segment (start 182.885 109.365) (end 182.885 112.55) (width 0.2) (layer "B.Cu") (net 5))
 (segment (start 156.305923 70.005923) (end 161.15 74.85) (width 0.2) (layer "F.Cu") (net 4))
 (segment (start 186.45 82.245318) (end 186.45 98.1) (width 0.2) (layer "F.Cu") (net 4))
 (segment (start 186.45 98.1) (end 182.000058 98.1) (width 0.2) (layer "F.Cu") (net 4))
 (segment (start 161.15 74.85) (end 182.5 74.85) (width 0.2) (layer "F.Cu") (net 4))
 (segment (start 191.344077 70.005923) (end 191.344077 77.351241) (width 0.2) (layer "F.Cu") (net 4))
 (segment (start 181.249 101.498942) (end 184.050058 104.3) (width 0.2) (layer "F.Cu") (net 4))
 (segment (start 191.344077 77.351241) (end 186.45 82.245318) (width 0.2) (layer "F.Cu") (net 4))
 (segment (start 181.249 98.851058) (end 181.249 101.498942) (width 0.2) (layer "F.Cu") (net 4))
 (segment (start 184.050058 104.3) (end 184.25 104.3) (width 0.2) (layer "F.Cu") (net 4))
 (segment (start 182.5 74.85) (end 187.344077 70.005923) (width 0.2) (layer "F.Cu") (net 4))
 (segment (start 187.344077 70.005923) (end 191.344077 70.005923) (width 0.2) (layer "F.Cu") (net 4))
 (segment (start 182.000058 98.1) (end 181.249 98.851058) (width 0.2) (layer "F.Cu") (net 4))
 (segment (start 152.805923 70.005923) (end 156.305923 70.005923) (width 0.2) (layer "F.Cu") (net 4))
 (via (at 184.25 104.3) (size 0.6) (drill 0.3) (layers "F.Cu" "B.Cu") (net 4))
 (segment (start 184.25 104.3) (end 180.15 104.3) (width 0.2) (layer "B.Cu") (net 4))
 (segment (start 180.15 104.3) (end 171.9 112.55) (width 0.2) (layer "B.Cu") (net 4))
 (segment (start 177.71 83.64) (end 185.955923 75.394077) (width 0.2) (layer "F.Cu") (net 1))
 (segment (start 177.71 86.85) (end 177.71 83.64) (width 0.2) (layer "F.Cu") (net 1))
 (segment (start 163.26 86.85) (end 163.26 80.46) (width 0.2) (layer "F.Cu") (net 3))
 (segment (start 163.26 80.46) (end 158.194077 75.394077) (width 0.2) (layer "F.Cu") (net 3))
 (segment (start 169.049999 99.5) (end 167.9 98.350001) (width 0.2) (layer "F.Cu") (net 2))
 (segment (start 167.9 98.350001) (end 167.9 97.85) (width 0.2) (layer "F.Cu") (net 2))
 (segment (start 169.049999 99.5) (end 175.55 99.500001) (width 0.2) (layer "F.Cu") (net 2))
 (segment (start 175.649999 99.500001) (end 176.7 98.45) (width 0.2) (layer "F.Cu") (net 2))
 (segment (start 175.55 99.500001) (end 175.649999 99.500001) (width 0.2) (layer "F.Cu") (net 2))
 (via (at 167.9 97.85) (size 0.6) (drill 0.3) (layers "F.Cu" "B.Cu") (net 2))
 (via (at 176.7 98.45) (size 0.6) (drill 0.3) (layers "F.Cu" "B.Cu") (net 2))
 (segment (start 180.25 94.9) (end 180.25 86.85) (width 0.2) (layer "B.Cu") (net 2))
 (segment (start 167.9 96.8) (end 165.8 94.7) (width 0.2) (layer "B.Cu") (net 2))
 (segment (start 176.7 98.45) (end 180.25 94.9) (width 0.2) (layer "B.Cu") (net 2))
 (segment (start 165.8 94.7) (end 165.8 86.85) (width 0.2) (layer "B.Cu") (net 2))
 (segment (start 167.9 97.85) (end 167.9 96.8) (width 0.2) (layer "B.Cu") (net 2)))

